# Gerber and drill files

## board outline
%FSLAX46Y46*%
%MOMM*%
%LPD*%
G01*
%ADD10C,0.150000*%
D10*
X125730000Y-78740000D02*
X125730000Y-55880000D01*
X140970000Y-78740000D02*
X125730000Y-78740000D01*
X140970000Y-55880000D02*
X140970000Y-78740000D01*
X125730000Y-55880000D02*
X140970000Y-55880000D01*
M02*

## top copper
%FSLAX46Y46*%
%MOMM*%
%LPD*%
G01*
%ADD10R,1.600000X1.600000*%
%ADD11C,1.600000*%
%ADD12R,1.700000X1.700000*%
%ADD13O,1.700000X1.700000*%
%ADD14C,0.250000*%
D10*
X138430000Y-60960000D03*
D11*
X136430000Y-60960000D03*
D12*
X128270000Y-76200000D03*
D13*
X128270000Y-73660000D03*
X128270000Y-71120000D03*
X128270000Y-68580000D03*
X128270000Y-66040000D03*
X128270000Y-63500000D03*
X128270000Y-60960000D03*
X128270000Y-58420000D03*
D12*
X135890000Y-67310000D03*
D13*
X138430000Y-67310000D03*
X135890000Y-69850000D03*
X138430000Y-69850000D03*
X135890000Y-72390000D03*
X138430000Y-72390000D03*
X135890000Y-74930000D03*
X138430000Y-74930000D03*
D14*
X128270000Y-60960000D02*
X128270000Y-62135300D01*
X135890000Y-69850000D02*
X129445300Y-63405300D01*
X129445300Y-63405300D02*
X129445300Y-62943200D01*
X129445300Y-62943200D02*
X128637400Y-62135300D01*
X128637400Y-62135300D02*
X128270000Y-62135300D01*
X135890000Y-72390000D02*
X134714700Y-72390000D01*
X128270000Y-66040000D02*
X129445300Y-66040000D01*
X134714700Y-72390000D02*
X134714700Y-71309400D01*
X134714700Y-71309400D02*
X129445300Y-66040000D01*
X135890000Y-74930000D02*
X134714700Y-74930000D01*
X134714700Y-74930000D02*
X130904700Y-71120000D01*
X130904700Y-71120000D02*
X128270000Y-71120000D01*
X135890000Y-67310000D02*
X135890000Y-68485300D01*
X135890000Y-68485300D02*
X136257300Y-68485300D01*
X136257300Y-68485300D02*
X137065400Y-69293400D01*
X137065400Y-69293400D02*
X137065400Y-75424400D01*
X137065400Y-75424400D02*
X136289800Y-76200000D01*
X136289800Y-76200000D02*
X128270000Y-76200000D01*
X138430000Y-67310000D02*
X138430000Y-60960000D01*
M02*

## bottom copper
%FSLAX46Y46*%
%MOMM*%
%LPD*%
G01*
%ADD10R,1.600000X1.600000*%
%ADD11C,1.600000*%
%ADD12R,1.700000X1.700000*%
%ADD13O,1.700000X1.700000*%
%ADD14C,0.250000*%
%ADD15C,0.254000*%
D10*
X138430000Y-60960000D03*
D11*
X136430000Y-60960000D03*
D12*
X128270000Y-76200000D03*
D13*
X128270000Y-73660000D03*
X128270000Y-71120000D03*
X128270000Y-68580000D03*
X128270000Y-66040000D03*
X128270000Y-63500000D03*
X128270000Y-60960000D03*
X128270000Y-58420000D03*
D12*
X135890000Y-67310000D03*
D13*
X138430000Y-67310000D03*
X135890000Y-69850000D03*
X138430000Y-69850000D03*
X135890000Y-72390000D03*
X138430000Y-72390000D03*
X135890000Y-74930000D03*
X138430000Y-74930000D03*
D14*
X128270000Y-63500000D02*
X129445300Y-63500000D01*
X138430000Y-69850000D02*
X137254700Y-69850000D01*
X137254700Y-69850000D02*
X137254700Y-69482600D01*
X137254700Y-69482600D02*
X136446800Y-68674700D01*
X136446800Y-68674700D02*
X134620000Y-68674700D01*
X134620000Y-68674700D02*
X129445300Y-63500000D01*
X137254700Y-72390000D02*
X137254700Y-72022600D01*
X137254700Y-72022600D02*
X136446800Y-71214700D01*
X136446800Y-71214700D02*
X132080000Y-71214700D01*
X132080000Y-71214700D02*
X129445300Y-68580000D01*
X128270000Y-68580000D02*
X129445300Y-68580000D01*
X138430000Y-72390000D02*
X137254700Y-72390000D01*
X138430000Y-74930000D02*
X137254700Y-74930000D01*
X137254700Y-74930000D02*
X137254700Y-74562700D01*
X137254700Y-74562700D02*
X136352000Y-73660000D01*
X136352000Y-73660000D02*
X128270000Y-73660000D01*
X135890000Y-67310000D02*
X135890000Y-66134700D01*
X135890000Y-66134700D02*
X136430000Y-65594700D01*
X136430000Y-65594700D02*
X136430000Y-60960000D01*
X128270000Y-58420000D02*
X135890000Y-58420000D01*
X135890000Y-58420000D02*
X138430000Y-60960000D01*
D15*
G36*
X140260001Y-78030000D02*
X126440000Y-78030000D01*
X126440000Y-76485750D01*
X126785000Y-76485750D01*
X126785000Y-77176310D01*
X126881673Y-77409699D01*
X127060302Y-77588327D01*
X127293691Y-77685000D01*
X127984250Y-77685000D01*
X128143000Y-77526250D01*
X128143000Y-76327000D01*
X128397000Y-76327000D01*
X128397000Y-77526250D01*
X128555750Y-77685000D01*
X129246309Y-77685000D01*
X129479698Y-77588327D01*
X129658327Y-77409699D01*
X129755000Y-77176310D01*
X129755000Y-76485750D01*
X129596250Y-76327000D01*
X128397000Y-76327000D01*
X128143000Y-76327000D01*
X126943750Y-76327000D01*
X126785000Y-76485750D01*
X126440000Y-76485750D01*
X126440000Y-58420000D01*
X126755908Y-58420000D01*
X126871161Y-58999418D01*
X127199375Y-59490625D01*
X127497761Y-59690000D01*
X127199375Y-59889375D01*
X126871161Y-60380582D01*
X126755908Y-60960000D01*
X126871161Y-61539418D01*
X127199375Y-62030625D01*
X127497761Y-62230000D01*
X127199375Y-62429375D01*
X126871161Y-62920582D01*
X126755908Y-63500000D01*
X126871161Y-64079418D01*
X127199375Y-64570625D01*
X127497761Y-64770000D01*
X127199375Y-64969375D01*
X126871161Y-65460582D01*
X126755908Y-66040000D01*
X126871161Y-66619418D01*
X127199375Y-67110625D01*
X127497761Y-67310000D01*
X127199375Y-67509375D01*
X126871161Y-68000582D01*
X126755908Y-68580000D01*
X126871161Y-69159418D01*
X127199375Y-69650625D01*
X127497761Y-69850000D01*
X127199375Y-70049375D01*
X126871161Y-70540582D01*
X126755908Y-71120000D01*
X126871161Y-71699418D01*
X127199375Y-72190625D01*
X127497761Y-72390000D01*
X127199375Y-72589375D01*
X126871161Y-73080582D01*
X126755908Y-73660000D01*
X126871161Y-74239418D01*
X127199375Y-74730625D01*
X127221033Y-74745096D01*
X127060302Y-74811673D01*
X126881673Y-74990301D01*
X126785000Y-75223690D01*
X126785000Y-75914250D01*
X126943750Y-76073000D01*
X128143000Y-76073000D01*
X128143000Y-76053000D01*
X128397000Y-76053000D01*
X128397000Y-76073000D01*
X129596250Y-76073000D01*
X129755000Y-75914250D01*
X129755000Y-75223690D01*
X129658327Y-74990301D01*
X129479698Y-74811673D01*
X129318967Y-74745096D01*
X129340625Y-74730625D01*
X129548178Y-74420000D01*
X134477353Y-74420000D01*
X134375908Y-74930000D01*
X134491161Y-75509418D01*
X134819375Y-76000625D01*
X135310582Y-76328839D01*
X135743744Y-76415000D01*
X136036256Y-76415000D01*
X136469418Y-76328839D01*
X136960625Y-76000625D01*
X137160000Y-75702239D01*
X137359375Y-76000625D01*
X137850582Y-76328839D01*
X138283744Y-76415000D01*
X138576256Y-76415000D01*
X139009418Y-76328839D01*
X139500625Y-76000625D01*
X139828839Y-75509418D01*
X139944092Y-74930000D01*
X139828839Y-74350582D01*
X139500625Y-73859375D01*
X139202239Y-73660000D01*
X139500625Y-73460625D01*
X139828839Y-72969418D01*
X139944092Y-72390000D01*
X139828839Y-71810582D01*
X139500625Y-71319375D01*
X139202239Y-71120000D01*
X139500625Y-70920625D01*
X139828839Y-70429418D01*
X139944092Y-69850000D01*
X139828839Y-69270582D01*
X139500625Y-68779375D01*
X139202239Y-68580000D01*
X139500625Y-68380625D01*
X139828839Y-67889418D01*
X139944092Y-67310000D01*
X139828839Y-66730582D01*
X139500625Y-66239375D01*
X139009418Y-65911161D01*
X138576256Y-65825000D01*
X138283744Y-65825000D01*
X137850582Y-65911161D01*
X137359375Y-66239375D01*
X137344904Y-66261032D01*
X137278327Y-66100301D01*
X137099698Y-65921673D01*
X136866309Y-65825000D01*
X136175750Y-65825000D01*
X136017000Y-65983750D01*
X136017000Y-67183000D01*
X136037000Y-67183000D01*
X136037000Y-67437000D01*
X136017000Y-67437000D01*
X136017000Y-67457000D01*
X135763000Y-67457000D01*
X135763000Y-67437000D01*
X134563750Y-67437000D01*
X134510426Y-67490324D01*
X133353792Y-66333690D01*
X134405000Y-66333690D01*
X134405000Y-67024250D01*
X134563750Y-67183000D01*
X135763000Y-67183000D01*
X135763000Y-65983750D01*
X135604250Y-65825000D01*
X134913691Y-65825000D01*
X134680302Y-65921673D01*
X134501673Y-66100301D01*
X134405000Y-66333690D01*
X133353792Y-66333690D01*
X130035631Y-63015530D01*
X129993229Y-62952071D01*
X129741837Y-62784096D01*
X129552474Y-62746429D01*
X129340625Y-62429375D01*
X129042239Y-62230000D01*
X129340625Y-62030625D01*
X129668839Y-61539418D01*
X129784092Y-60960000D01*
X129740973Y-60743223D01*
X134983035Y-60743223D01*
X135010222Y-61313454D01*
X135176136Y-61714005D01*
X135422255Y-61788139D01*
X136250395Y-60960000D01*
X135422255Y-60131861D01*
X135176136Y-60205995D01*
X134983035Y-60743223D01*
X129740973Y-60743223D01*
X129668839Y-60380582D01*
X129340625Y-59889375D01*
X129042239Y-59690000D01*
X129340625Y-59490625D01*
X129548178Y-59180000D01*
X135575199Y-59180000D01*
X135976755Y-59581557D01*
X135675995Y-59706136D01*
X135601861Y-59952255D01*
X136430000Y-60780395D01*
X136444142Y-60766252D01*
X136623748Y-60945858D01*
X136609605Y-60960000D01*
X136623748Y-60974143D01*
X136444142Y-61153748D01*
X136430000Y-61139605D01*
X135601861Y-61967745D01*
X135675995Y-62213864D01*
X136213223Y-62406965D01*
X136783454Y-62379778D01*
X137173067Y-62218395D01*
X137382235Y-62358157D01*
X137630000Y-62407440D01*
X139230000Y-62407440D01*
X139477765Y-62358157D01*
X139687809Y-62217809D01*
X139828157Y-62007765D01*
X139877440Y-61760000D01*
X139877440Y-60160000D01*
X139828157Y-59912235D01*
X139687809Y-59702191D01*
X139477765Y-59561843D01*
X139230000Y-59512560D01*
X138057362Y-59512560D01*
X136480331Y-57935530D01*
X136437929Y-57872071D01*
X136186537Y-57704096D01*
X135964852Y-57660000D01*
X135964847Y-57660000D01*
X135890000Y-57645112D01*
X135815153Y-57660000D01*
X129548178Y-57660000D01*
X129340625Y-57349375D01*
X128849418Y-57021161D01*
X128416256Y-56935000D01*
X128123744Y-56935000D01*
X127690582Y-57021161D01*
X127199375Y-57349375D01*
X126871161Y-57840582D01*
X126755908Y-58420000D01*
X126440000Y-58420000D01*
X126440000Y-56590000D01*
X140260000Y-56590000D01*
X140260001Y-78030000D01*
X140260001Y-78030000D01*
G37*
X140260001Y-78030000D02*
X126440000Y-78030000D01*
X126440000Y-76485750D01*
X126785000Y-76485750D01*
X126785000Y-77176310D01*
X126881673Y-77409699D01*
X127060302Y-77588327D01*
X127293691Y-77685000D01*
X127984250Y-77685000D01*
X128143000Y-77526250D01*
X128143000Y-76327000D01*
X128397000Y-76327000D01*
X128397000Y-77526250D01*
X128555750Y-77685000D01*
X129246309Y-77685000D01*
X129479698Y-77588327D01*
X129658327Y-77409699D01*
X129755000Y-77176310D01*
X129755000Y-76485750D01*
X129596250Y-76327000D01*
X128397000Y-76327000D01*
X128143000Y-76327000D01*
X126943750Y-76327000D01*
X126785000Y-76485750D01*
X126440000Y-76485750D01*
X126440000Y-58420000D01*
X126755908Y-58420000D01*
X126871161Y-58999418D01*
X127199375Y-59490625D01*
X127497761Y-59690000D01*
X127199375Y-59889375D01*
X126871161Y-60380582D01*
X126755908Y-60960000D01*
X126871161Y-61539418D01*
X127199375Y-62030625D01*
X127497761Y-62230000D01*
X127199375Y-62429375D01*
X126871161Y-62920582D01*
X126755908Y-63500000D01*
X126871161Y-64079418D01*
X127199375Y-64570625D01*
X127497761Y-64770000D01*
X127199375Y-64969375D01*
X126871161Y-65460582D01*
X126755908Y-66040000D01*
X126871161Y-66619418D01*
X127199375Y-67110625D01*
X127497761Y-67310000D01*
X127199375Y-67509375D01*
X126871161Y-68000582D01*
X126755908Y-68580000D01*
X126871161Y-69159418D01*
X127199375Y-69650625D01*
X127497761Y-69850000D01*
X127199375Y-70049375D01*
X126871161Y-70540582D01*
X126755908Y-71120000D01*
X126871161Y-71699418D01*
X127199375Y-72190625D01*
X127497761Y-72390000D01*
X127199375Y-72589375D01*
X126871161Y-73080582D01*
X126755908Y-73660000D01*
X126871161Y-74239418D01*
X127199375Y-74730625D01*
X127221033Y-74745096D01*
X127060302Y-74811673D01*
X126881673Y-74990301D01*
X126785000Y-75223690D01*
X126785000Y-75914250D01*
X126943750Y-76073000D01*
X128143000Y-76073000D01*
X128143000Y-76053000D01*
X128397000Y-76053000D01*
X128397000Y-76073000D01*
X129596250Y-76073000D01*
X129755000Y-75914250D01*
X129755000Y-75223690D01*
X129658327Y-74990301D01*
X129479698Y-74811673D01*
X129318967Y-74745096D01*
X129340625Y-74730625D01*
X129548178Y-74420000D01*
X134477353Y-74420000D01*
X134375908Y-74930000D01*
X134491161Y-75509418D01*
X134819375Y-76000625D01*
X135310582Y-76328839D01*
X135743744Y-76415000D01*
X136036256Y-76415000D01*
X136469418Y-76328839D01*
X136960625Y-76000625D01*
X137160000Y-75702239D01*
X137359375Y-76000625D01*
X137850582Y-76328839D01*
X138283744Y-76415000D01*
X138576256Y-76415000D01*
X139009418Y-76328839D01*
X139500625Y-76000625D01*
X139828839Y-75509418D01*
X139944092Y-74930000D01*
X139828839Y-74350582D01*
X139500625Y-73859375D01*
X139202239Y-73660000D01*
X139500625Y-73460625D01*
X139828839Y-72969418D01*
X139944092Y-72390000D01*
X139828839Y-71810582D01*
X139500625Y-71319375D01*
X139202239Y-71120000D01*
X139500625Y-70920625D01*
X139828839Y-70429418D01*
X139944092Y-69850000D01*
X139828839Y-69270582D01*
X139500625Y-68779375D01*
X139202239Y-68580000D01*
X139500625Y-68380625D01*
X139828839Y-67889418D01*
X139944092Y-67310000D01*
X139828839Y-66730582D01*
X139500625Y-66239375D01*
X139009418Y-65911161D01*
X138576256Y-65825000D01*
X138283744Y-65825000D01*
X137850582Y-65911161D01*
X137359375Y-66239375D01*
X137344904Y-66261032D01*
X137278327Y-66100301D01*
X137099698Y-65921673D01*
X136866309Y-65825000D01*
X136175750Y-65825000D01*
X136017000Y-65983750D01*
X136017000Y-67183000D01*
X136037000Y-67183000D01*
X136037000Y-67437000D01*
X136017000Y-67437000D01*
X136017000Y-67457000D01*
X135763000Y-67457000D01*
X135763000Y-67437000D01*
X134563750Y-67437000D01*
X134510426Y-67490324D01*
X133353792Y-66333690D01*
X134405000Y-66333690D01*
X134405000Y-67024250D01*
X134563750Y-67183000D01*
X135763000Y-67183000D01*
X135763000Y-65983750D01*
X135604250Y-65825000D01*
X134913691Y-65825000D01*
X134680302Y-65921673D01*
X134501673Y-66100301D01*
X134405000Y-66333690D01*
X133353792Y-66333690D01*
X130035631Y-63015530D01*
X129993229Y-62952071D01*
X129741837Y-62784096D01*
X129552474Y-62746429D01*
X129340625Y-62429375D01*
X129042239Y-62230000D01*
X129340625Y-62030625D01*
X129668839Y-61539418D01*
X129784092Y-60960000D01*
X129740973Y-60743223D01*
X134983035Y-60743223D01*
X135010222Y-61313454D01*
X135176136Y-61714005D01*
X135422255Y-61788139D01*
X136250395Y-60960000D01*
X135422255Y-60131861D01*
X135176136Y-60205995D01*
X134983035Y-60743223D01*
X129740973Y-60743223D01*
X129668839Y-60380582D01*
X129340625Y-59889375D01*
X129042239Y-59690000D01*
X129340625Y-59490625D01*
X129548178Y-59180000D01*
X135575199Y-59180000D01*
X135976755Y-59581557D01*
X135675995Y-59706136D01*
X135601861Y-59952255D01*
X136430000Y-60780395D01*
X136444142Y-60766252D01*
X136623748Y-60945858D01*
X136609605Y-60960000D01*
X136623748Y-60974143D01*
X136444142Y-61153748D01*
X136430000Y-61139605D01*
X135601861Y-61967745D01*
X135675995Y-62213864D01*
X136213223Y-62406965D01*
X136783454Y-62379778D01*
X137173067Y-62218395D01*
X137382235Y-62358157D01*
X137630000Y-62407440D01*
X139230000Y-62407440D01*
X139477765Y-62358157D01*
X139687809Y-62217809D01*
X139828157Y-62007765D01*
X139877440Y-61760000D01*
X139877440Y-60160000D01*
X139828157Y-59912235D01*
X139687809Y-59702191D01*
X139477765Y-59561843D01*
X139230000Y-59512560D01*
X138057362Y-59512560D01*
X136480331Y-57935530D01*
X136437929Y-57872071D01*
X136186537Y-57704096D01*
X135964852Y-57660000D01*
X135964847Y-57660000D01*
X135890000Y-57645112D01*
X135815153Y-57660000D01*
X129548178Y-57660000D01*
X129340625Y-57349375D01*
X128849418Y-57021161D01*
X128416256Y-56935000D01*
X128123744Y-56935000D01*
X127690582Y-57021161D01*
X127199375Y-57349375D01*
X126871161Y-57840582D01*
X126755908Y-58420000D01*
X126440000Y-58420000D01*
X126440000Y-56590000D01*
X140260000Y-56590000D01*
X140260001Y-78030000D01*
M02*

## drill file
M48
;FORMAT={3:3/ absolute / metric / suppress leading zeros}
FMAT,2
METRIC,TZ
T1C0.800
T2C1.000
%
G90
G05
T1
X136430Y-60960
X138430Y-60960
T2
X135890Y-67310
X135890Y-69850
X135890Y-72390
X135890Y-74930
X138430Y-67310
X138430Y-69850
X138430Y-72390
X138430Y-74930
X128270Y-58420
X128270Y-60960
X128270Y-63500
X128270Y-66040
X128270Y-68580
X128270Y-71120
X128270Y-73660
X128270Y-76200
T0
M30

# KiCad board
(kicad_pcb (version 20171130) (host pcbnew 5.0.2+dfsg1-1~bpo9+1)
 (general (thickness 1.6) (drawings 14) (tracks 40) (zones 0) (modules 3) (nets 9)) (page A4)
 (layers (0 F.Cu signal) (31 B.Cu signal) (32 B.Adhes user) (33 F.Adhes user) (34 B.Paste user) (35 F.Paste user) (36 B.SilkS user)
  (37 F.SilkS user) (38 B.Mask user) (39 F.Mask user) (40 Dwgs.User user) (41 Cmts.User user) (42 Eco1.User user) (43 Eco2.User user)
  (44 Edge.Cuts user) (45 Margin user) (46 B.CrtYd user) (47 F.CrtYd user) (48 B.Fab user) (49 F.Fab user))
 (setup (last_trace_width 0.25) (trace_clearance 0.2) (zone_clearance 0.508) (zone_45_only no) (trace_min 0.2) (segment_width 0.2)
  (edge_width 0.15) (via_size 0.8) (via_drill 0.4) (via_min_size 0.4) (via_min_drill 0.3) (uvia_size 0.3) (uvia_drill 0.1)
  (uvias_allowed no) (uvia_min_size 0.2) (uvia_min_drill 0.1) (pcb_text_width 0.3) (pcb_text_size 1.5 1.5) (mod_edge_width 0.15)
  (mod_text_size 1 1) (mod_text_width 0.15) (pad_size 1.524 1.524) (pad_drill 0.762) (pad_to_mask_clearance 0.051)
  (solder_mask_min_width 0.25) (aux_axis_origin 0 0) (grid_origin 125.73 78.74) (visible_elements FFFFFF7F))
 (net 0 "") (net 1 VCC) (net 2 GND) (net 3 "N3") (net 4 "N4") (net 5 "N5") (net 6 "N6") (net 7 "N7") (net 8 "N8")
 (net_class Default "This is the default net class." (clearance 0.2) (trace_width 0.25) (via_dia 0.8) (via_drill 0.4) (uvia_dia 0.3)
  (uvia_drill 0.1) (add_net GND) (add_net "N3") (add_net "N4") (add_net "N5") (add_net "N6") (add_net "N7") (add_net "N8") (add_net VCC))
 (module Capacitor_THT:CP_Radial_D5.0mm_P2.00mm (layer F.Cu) (at 138.43 60.96 180)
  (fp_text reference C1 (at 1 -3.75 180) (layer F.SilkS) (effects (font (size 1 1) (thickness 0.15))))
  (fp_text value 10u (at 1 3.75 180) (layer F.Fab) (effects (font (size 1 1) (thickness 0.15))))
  (pad 1 thru_hole rect (at 0 0 180) (size 1.6 1.6) (drill 0.8) (layers *.Cu *.Mask) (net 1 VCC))
  (pad 2 thru_hole circle (at 2 0 180) (size 1.6 1.6) (drill 0.8) (layers *.Cu *.Mask) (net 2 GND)))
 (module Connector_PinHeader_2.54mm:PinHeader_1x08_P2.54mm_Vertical (layer B.Cu) (at 128.27 76.2)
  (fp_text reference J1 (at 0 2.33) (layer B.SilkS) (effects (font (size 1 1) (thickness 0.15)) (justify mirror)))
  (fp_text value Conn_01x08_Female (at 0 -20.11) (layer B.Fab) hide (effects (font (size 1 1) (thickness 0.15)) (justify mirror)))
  (pad 1 thru_hole rect (at 0 0) (size 1.7 1.7) (drill 1) (layers *.Cu *.Mask) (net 2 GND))
  (pad 2 thru_hole oval (at 0 -2.54) (size 1.7 1.7) (drill 1) (layers *.Cu *.Mask) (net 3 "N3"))
  (pad 3 thru_hole oval (at 0 -5.08) (size 1.7 1.7) (drill 1) (layers *.Cu *.Mask) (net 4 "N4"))
  (pad 4 thru_hole oval (at 0 -7.62) (size 1.7 1.7) (drill 1) (layers *.Cu *.Mask) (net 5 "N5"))
  (pad 5 thru_hole oval (at 0 -10.16) (size 1.7 1.7) (drill 1) (layers *.Cu *.Mask) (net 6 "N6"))
  (pad 6 thru_hole oval (at 0 -12.7) (size 1.7 1.7) (drill 1) (layers *.Cu *.Mask) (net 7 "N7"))
  (pad 7 thru_hole oval (at 0 -15.24) (size 1.7 1.7) (drill 1) (layers *.Cu *.Mask) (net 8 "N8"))
  (pad 8 thru_hole oval (at 0 -17.78) (size 1.7 1.7) (drill 1) (layers *.Cu *.Mask) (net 1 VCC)))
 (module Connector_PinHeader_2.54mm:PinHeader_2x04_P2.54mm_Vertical (layer F.Cu) (at 135.89 67.31)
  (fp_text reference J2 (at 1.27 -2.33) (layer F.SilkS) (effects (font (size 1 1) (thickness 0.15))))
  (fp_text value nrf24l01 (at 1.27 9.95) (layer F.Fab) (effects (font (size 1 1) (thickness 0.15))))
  (pad 1 thru_hole rect (at 0 0) (size 1.7 1.7) (drill 1) (layers *.Cu *.Mask) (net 2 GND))
  (pad 2 thru_hole oval (at 2.54 0) (size 1.7 1.7) (drill 1) (layers *.Cu *.Mask) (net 1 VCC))
  (pad 3 thru_hole oval (at 0 2.54) (size 1.7 1.7) (drill 1) (layers *.Cu *.Mask) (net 8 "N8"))
  (pad 4 thru_hole oval (at 2.54 2.54) (size 1.7 1.7) (drill 1) (layers *.Cu *.Mask) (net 7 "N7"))
  (pad 5 thru_hole oval (at 0 5.08) (size 1.7 1.7) (drill 1) (layers *.Cu *.Mask) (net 6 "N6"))
  (pad 6 thru_hole oval (at 2.54 5.08) (size 1.7 1.7) (drill 1) (layers *.Cu *.Mask) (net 5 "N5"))
  (pad 7 thru_hole oval (at 0 7.62) (size 1.7 1.7) (drill 1) (layers *.Cu *.Mask) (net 4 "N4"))
  (pad 8 thru_hole oval (at 2.54 7.62) (size 1.7 1.7) (drill 1) (layers *.Cu *.Mask) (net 3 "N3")))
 (gr_line (start 125.73 78.74) (end 125.73 55.88) (layer Edge.Cuts) (width 0.15))
 (gr_line (start 140.97 78.74) (end 125.73 78.74) (layer Edge.Cuts) (width 0.15))
 (gr_line (start 140.97 55.88) (end 140.97 78.74) (layer Edge.Cuts) (width 0.15))
 (gr_line (start 125.73 55.88) (end 140.97 55.88) (layer Edge.Cuts) (width 0.15))
 (segment (start 135.89 67.31) (end 135.89 66.1347) (width 0.25) (layer B.Cu) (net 2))
 (segment (start 135.89 66.1347) (end 136.43 65.5947) (width 0.25) (layer B.Cu) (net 2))
 (segment (start 136.43 65.5947) (end 136.43 60.96) (width 0.25) (layer B.Cu) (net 2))
 (segment (start 135.89 67.31) (end 135.89 68.4853) (width 0.25) (layer F.Cu) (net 2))
 (segment (start 135.89 68.4853) (end 136.2573 68.4853) (width 0.25) (layer F.Cu) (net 2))
 (segment (start 136.2573 68.4853) (end 137.0654 69.2934) (width 0.25) (layer F.Cu) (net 2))
 (segment (start 137.0654 69.2934) (end 137.0654 75.4244) (width 0.25) (layer F.Cu) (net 2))
 (segment (start 137.0654 75.4244) (end 136.2898 76.2) (width 0.25) (layer F.Cu) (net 2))
 (segment (start 136.2898 76.2) (end 128.27 76.2) (width 0.25) (layer F.Cu) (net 2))
 (segment (start 128.27 58.42) (end 135.89 58.42) (width 0.25) (layer B.Cu) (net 1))
 (segment (start 135.89 58.42) (end 138.43 60.96) (width 0.25) (layer B.Cu) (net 1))
 (segment (start 138.43 67.31) (end 138.43 60.96) (width 0.25) (layer F.Cu) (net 1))
 (segment (start 128.27 60.96) (end 128.27 62.1353) (width 0.25) (layer F.Cu) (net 8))
 (segment (start 135.89 69.85) (end 129.4453 63.4053) (width 0.25) (layer F.Cu) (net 8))
 (segment (start 129.4453 63.4053) (end 129.4453 62.9432) (width 0.25) (layer F.Cu) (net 8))
 (segment (start 129.4453 62.9432) (end 128.6374 62.1353) (width 0.25) (layer F.Cu) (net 8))
 (segment (start 128.6374 62.1353) (end 128.27 62.1353) (width 0.25) (layer F.Cu) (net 8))
 (segment (start 128.27 63.5) (end 129.4453 63.5) (width 0.25) (layer B.Cu) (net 7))
 (segment (start 138.43 69.85) (end 137.2547 69.85) (width 0.25) (layer B.Cu) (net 7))
 (segment (start 137.2547 69.85) (end 137.2547 69.4826) (width 0.25) (layer B.Cu) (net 7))
 (segment (start 137.2547 69.4826) (end 136.4468 68.6747) (width 0.25) (layer B.Cu) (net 7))
 (segment (start 136.4468 68.6747) (end 134.62 68.6747) (width 0.25) (layer B.Cu) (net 7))
 (segment (start 134.62 68.6747) (end 129.4453 63.5) (width 0.25) (layer B.Cu) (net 7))
 (segment (start 135.89 72.39) (end 134.7147 72.39) (width 0.25) (layer F.Cu) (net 6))
 (segment (start 128.27 66.04) (end 129.4453 66.04) (width 0.25) (layer F.Cu) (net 6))
 (segment (start 134.7147 72.39) (end 134.7147 71.3094) (width 0.25) (layer F.Cu) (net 6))
 (segment (start 134.7147 71.3094) (end 129.4453 66.04) (width 0.25) (layer F.Cu) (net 6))
 (segment (start 137.2547 72.39) (end 137.2547 72.0226) (width 0.25) (layer B.Cu) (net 5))
 (segment (start 137.2547 72.0226) (end 136.4468 71.2147) (width 0.25) (layer B.Cu) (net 5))
 (segment (start 136.4468 71.2147) (end 132.08 71.2147) (width 0.25) (layer B.Cu) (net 5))
 (segment (start 132.08 71.2147) (end 129.4453 68.58) (width 0.25) (layer B.Cu) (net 5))
 (segment (start 128.27 68.58) (end 129.4453 68.58) (width 0.25) (layer B.Cu) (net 5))
 (segment (start 138.43 72.39) (end 137.2547 72.39) (width 0.25) (layer B.Cu) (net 5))
 (segment (start 135.89 74.93) (end 134.7147 74.93) (width 0.25) (layer F.Cu) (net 4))
 (segment (start 134.7147 74.93) (end 130.9047 71.12) (width 0.25) (layer F.Cu) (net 4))
 (segment (start 130.9047 71.12) (end 128.27 71.12) (width 0.25) (layer F.Cu) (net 4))
 (segment (start 138.43 74.93) (end 137.2547 74.93) (width 0.25) (layer B.Cu) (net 3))
 (segment (start 137.2547 74.93) (end 137.2547 74.5627) (width 0.25) (layer B.Cu) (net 3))
 (segment (start 137.2547 74.5627) (end 136.352 73.66) (width 0.25) (layer B.Cu) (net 3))
 (segment (start 136.352 73.66) (end 128.27 73.66) (width 0.25) (layer B.Cu) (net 3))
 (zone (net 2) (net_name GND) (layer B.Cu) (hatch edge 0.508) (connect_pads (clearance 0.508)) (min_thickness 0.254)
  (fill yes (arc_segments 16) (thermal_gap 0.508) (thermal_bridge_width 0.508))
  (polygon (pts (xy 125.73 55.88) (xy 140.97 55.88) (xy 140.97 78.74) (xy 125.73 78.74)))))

